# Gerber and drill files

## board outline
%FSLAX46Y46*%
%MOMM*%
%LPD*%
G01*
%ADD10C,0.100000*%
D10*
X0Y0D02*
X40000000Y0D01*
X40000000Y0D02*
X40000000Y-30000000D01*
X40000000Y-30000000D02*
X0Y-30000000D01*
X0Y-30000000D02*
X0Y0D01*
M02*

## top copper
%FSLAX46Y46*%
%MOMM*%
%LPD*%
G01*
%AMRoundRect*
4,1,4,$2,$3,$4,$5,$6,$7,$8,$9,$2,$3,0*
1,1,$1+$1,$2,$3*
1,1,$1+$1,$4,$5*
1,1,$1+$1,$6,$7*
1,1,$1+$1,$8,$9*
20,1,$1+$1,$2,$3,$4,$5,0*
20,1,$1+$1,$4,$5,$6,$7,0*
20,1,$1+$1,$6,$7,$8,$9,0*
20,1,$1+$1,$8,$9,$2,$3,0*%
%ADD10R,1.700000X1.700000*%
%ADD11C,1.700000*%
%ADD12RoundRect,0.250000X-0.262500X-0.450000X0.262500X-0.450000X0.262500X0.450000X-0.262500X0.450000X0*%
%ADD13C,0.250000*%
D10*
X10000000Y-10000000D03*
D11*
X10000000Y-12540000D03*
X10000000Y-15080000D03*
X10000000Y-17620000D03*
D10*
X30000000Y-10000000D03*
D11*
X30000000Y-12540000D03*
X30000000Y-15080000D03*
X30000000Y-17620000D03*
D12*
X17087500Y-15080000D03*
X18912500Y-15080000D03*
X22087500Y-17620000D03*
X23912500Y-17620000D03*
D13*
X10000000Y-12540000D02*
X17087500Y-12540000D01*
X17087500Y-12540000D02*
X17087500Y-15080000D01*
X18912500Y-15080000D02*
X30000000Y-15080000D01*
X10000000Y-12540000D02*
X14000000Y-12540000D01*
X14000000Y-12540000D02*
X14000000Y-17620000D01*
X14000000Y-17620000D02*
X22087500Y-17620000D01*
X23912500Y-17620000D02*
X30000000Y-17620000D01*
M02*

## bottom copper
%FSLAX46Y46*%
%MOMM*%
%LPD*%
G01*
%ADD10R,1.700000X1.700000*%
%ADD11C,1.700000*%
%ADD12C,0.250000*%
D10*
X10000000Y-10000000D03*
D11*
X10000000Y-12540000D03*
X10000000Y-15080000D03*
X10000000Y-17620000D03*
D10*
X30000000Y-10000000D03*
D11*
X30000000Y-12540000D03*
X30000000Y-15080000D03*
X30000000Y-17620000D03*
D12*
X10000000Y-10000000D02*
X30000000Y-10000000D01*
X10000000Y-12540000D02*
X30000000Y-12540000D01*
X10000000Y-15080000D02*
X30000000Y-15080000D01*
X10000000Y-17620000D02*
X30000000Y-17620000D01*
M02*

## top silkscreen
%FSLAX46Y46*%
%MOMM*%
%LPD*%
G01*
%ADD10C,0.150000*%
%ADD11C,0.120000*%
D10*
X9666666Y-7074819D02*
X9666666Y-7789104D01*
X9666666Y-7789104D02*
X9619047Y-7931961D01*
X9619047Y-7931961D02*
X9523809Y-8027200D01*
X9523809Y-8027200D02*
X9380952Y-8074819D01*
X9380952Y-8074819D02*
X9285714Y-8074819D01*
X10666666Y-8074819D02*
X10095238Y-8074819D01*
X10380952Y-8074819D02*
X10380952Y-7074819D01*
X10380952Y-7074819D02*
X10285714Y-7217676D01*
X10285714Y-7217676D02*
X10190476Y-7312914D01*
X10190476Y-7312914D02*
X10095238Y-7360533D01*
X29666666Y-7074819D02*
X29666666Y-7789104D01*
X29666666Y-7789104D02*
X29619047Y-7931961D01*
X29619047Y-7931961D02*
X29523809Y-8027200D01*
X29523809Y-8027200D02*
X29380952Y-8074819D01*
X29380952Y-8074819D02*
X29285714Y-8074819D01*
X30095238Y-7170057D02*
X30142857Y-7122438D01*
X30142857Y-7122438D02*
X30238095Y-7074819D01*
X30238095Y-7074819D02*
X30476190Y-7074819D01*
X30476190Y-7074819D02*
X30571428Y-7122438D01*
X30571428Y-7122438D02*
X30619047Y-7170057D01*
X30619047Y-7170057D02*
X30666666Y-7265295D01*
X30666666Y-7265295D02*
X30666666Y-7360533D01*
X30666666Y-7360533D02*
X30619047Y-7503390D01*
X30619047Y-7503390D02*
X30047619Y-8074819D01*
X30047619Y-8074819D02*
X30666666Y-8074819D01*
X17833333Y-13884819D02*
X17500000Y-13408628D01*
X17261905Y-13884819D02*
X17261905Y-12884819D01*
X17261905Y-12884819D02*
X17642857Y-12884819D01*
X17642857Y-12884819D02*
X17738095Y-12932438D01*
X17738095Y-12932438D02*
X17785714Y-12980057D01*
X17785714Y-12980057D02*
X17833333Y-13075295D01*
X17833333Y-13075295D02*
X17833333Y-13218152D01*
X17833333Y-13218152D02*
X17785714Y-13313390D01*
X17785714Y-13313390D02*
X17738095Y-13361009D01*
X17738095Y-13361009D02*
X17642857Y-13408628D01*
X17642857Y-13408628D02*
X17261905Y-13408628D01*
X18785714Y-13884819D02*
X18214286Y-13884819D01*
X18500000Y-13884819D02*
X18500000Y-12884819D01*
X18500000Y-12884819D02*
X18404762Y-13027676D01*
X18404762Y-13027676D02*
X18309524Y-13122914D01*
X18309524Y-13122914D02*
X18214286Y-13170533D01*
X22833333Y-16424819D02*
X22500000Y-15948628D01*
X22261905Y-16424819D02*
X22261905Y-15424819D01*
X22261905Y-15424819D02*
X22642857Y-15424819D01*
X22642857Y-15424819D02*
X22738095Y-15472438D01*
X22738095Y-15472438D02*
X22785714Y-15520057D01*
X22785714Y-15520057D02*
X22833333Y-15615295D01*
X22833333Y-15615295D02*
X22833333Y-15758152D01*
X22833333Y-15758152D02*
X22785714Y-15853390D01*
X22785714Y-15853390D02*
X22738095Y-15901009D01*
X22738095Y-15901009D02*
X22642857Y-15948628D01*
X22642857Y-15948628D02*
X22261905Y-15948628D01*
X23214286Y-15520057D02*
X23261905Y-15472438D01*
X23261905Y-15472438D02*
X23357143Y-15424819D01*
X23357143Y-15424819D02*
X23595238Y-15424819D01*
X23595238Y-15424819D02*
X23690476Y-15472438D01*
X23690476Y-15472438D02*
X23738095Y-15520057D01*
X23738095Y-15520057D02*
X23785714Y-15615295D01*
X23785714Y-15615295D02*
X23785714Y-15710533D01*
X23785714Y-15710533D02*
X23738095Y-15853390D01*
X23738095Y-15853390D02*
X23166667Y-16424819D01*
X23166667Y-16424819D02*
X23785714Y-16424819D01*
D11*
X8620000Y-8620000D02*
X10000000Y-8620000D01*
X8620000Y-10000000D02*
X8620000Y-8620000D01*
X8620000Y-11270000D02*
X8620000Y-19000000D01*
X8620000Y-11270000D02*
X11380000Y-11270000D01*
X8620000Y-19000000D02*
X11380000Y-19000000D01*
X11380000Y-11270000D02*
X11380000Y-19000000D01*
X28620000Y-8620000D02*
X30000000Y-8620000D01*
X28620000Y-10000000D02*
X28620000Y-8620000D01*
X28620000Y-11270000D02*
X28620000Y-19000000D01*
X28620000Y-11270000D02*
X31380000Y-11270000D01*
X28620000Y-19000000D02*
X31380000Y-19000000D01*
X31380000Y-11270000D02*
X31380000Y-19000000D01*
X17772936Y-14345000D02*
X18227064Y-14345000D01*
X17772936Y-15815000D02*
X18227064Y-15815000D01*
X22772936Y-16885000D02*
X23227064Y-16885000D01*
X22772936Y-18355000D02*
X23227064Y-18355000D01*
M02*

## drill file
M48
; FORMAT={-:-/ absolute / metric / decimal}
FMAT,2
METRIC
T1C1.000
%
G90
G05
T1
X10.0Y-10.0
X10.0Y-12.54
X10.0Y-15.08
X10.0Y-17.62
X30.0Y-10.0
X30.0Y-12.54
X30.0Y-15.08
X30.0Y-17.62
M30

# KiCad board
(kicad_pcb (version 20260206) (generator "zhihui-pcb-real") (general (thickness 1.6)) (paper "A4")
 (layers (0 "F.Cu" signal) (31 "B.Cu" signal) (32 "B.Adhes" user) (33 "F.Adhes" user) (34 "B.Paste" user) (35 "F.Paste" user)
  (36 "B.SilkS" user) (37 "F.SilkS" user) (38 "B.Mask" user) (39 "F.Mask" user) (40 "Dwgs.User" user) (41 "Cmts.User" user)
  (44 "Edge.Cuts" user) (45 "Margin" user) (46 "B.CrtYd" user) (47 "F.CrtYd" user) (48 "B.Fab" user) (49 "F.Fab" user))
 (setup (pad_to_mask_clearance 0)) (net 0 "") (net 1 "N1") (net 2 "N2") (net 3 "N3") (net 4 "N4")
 (gr_line (start 0 0) (end 40 0) (stroke (width 0.1) (type default)) (layer "Edge.Cuts"))
 (gr_line (start 40 0) (end 40 30) (stroke (width 0.1) (type default)) (layer "Edge.Cuts"))
 (gr_line (start 40 30) (end 0 30) (stroke (width 0.1) (type default)) (layer "Edge.Cuts"))
 (gr_line (start 0 30) (end 0 0) (stroke (width 0.1) (type default)) (layer "Edge.Cuts"))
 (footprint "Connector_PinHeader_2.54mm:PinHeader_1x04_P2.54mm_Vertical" (layer "F.Cu")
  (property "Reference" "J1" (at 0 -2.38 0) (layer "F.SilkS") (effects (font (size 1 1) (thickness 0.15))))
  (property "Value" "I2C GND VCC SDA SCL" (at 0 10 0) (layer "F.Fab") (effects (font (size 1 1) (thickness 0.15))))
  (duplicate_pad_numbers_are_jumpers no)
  (fp_line (start -1.38 -1.38) (end 0 -1.38) (stroke (width 0.12) (type solid)) (layer "F.SilkS"))
  (fp_line (start -1.38 0) (end -1.38 -1.38) (stroke (width 0.12) (type solid)) (layer "F.SilkS"))
  (fp_line (start -1.38 1.27) (end -1.38 9) (stroke (width 0.12) (type solid)) (layer "F.SilkS"))
  (fp_line (start -1.38 1.27) (end 1.38 1.27) (stroke (width 0.12) (type solid)) (layer "F.SilkS"))
  (fp_line (start -1.38 9) (end 1.38 9) (stroke (width 0.12) (type solid)) (layer "F.SilkS"))
  (fp_line (start 1.38 1.27) (end 1.38 9) (stroke (width 0.12) (type solid)) (layer "F.SilkS"))
  (pad "1" thru_hole rect (at 0 0) (size 1.7 1.7) (drill 1) (layers "*.Cu" "*.Mask") (remove_unused_layers no) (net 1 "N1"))
  (pad "2" thru_hole circle (at 0 2.54) (size 1.7 1.7) (drill 1) (layers "*.Cu" "*.Mask") (remove_unused_layers no) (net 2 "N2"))
  (pad "3" thru_hole circle (at 0 5.08) (size 1.7 1.7) (drill 1) (layers "*.Cu" "*.Mask") (remove_unused_layers no) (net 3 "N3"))
  (pad "4" thru_hole circle (at 0 7.62) (size 1.7 1.7) (drill 1) (layers "*.Cu" "*.Mask") (remove_unused_layers no) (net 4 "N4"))
  (at 10 10 0))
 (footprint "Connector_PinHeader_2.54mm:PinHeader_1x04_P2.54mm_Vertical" (layer "F.Cu")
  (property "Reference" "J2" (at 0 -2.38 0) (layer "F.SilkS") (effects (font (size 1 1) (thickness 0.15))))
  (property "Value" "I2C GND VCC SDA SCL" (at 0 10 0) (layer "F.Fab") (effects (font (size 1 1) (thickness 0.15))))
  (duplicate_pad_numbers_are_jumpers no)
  (fp_line (start -1.38 -1.38) (end 0 -1.38) (stroke (width 0.12) (type solid)) (layer "F.SilkS"))
  (fp_line (start -1.38 0) (end -1.38 -1.38) (stroke (width 0.12) (type solid)) (layer "F.SilkS"))
  (fp_line (start -1.38 1.27) (end -1.38 9) (stroke (width 0.12) (type solid)) (layer "F.SilkS"))
  (fp_line (start -1.38 1.27) (end 1.38 1.27) (stroke (width 0.12) (type solid)) (layer "F.SilkS"))
  (fp_line (start -1.38 9) (end 1.38 9) (stroke (width 0.12) (type solid)) (layer "F.SilkS"))
  (fp_line (start 1.38 1.27) (end 1.38 9) (stroke (width 0.12) (type solid)) (layer "F.SilkS"))
  (pad "1" thru_hole rect (at 0 0) (size 1.7 1.7) (drill 1) (layers "*.Cu" "*.Mask") (remove_unused_layers no) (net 1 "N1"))
  (pad "2" thru_hole circle (at 0 2.54) (size 1.7 1.7) (drill 1) (layers "*.Cu" "*.Mask") (remove_unused_layers no) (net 2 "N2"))
  (pad "3" thru_hole circle (at 0 5.08) (size 1.7 1.7) (drill 1) (layers "*.Cu" "*.Mask") (remove_unused_layers no) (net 3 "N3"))
  (pad "4" thru_hole circle (at 0 7.62) (size 1.7 1.7) (drill 1) (layers "*.Cu" "*.Mask") (remove_unused_layers no) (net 4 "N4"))
  (at 30 10 0))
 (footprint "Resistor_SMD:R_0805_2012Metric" (layer "F.Cu")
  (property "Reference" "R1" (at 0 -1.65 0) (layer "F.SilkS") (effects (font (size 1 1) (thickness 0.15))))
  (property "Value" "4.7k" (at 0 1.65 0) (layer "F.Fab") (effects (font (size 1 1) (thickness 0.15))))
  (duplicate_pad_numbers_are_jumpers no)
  (fp_line (start -0.227064 -0.735) (end 0.227064 -0.735) (stroke (width 0.12) (type solid)) (layer "F.SilkS"))
  (fp_line (start -0.227064 0.735) (end 0.227064 0.735) (stroke (width 0.12) (type solid)) (layer "F.SilkS"))
  (pad "1" smd roundrect (at -0.9125 0) (size 1.025 1.4) (layers "F.Cu" "F.Mask" "F.Paste") (roundrect_rratio 0.243902) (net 2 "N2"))
  (pad "2" smd roundrect (at 0.9125 0) (size 1.025 1.4) (layers "F.Cu" "F.Mask" "F.Paste") (roundrect_rratio 0.243902) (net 3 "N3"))
  (at 18 15.08 0))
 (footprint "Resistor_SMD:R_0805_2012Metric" (layer "F.Cu")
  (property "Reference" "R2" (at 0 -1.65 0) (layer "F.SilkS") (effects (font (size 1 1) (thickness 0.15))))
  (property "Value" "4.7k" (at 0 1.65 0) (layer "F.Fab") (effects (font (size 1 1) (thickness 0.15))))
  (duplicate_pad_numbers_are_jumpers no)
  (fp_line (start -0.227064 -0.735) (end 0.227064 -0.735) (stroke (width 0.12) (type solid)) (layer "F.SilkS"))
  (fp_line (start -0.227064 0.735) (end 0.227064 0.735) (stroke (width 0.12) (type solid)) (layer "F.SilkS"))
  (pad "1" smd roundrect (at -0.9125 0) (size 1.025 1.4) (layers "F.Cu" "F.Mask" "F.Paste") (roundrect_rratio 0.243902) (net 2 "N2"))
  (pad "2" smd roundrect (at 0.9125 0) (size 1.025 1.4) (layers "F.Cu" "F.Mask" "F.Paste") (roundrect_rratio 0.243902) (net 4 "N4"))
  (at 23 17.62 0))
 (segment (start 10 10) (end 30 10) (width 0.25) (layer "B.Cu") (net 1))
 (segment (start 10 12.54) (end 30 12.54) (width 0.25) (layer "B.Cu") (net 2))
 (segment (start 10 15.08) (end 30 15.08) (width 0.25) (layer "B.Cu") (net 3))
 (segment (start 10 17.62) (end 30 17.62) (width 0.25) (layer "B.Cu") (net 4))
 (segment (start 10 12.54) (end 17.0875 12.54) (width 0.25) (layer "F.Cu") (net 2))
 (segment (start 17.0875 12.54) (end 17.0875 15.08) (width 0.25) (layer "F.Cu") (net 2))
 (segment (start 18.9125 15.08) (end 30 15.08) (width 0.25) (layer "F.Cu") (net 3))
 (segment (start 10 12.54) (end 14 12.54) (width 0.25) (layer "F.Cu") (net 2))
 (segment (start 14 12.54) (end 14 17.62) (width 0.25) (layer "F.Cu") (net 2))
 (segment (start 14 17.62) (end 22.0875 17.62) (width 0.25) (layer "F.Cu") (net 2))
 (segment (start 23.9125 17.62) (end 30 17.62) (width 0.25) (layer "F.Cu") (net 4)))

